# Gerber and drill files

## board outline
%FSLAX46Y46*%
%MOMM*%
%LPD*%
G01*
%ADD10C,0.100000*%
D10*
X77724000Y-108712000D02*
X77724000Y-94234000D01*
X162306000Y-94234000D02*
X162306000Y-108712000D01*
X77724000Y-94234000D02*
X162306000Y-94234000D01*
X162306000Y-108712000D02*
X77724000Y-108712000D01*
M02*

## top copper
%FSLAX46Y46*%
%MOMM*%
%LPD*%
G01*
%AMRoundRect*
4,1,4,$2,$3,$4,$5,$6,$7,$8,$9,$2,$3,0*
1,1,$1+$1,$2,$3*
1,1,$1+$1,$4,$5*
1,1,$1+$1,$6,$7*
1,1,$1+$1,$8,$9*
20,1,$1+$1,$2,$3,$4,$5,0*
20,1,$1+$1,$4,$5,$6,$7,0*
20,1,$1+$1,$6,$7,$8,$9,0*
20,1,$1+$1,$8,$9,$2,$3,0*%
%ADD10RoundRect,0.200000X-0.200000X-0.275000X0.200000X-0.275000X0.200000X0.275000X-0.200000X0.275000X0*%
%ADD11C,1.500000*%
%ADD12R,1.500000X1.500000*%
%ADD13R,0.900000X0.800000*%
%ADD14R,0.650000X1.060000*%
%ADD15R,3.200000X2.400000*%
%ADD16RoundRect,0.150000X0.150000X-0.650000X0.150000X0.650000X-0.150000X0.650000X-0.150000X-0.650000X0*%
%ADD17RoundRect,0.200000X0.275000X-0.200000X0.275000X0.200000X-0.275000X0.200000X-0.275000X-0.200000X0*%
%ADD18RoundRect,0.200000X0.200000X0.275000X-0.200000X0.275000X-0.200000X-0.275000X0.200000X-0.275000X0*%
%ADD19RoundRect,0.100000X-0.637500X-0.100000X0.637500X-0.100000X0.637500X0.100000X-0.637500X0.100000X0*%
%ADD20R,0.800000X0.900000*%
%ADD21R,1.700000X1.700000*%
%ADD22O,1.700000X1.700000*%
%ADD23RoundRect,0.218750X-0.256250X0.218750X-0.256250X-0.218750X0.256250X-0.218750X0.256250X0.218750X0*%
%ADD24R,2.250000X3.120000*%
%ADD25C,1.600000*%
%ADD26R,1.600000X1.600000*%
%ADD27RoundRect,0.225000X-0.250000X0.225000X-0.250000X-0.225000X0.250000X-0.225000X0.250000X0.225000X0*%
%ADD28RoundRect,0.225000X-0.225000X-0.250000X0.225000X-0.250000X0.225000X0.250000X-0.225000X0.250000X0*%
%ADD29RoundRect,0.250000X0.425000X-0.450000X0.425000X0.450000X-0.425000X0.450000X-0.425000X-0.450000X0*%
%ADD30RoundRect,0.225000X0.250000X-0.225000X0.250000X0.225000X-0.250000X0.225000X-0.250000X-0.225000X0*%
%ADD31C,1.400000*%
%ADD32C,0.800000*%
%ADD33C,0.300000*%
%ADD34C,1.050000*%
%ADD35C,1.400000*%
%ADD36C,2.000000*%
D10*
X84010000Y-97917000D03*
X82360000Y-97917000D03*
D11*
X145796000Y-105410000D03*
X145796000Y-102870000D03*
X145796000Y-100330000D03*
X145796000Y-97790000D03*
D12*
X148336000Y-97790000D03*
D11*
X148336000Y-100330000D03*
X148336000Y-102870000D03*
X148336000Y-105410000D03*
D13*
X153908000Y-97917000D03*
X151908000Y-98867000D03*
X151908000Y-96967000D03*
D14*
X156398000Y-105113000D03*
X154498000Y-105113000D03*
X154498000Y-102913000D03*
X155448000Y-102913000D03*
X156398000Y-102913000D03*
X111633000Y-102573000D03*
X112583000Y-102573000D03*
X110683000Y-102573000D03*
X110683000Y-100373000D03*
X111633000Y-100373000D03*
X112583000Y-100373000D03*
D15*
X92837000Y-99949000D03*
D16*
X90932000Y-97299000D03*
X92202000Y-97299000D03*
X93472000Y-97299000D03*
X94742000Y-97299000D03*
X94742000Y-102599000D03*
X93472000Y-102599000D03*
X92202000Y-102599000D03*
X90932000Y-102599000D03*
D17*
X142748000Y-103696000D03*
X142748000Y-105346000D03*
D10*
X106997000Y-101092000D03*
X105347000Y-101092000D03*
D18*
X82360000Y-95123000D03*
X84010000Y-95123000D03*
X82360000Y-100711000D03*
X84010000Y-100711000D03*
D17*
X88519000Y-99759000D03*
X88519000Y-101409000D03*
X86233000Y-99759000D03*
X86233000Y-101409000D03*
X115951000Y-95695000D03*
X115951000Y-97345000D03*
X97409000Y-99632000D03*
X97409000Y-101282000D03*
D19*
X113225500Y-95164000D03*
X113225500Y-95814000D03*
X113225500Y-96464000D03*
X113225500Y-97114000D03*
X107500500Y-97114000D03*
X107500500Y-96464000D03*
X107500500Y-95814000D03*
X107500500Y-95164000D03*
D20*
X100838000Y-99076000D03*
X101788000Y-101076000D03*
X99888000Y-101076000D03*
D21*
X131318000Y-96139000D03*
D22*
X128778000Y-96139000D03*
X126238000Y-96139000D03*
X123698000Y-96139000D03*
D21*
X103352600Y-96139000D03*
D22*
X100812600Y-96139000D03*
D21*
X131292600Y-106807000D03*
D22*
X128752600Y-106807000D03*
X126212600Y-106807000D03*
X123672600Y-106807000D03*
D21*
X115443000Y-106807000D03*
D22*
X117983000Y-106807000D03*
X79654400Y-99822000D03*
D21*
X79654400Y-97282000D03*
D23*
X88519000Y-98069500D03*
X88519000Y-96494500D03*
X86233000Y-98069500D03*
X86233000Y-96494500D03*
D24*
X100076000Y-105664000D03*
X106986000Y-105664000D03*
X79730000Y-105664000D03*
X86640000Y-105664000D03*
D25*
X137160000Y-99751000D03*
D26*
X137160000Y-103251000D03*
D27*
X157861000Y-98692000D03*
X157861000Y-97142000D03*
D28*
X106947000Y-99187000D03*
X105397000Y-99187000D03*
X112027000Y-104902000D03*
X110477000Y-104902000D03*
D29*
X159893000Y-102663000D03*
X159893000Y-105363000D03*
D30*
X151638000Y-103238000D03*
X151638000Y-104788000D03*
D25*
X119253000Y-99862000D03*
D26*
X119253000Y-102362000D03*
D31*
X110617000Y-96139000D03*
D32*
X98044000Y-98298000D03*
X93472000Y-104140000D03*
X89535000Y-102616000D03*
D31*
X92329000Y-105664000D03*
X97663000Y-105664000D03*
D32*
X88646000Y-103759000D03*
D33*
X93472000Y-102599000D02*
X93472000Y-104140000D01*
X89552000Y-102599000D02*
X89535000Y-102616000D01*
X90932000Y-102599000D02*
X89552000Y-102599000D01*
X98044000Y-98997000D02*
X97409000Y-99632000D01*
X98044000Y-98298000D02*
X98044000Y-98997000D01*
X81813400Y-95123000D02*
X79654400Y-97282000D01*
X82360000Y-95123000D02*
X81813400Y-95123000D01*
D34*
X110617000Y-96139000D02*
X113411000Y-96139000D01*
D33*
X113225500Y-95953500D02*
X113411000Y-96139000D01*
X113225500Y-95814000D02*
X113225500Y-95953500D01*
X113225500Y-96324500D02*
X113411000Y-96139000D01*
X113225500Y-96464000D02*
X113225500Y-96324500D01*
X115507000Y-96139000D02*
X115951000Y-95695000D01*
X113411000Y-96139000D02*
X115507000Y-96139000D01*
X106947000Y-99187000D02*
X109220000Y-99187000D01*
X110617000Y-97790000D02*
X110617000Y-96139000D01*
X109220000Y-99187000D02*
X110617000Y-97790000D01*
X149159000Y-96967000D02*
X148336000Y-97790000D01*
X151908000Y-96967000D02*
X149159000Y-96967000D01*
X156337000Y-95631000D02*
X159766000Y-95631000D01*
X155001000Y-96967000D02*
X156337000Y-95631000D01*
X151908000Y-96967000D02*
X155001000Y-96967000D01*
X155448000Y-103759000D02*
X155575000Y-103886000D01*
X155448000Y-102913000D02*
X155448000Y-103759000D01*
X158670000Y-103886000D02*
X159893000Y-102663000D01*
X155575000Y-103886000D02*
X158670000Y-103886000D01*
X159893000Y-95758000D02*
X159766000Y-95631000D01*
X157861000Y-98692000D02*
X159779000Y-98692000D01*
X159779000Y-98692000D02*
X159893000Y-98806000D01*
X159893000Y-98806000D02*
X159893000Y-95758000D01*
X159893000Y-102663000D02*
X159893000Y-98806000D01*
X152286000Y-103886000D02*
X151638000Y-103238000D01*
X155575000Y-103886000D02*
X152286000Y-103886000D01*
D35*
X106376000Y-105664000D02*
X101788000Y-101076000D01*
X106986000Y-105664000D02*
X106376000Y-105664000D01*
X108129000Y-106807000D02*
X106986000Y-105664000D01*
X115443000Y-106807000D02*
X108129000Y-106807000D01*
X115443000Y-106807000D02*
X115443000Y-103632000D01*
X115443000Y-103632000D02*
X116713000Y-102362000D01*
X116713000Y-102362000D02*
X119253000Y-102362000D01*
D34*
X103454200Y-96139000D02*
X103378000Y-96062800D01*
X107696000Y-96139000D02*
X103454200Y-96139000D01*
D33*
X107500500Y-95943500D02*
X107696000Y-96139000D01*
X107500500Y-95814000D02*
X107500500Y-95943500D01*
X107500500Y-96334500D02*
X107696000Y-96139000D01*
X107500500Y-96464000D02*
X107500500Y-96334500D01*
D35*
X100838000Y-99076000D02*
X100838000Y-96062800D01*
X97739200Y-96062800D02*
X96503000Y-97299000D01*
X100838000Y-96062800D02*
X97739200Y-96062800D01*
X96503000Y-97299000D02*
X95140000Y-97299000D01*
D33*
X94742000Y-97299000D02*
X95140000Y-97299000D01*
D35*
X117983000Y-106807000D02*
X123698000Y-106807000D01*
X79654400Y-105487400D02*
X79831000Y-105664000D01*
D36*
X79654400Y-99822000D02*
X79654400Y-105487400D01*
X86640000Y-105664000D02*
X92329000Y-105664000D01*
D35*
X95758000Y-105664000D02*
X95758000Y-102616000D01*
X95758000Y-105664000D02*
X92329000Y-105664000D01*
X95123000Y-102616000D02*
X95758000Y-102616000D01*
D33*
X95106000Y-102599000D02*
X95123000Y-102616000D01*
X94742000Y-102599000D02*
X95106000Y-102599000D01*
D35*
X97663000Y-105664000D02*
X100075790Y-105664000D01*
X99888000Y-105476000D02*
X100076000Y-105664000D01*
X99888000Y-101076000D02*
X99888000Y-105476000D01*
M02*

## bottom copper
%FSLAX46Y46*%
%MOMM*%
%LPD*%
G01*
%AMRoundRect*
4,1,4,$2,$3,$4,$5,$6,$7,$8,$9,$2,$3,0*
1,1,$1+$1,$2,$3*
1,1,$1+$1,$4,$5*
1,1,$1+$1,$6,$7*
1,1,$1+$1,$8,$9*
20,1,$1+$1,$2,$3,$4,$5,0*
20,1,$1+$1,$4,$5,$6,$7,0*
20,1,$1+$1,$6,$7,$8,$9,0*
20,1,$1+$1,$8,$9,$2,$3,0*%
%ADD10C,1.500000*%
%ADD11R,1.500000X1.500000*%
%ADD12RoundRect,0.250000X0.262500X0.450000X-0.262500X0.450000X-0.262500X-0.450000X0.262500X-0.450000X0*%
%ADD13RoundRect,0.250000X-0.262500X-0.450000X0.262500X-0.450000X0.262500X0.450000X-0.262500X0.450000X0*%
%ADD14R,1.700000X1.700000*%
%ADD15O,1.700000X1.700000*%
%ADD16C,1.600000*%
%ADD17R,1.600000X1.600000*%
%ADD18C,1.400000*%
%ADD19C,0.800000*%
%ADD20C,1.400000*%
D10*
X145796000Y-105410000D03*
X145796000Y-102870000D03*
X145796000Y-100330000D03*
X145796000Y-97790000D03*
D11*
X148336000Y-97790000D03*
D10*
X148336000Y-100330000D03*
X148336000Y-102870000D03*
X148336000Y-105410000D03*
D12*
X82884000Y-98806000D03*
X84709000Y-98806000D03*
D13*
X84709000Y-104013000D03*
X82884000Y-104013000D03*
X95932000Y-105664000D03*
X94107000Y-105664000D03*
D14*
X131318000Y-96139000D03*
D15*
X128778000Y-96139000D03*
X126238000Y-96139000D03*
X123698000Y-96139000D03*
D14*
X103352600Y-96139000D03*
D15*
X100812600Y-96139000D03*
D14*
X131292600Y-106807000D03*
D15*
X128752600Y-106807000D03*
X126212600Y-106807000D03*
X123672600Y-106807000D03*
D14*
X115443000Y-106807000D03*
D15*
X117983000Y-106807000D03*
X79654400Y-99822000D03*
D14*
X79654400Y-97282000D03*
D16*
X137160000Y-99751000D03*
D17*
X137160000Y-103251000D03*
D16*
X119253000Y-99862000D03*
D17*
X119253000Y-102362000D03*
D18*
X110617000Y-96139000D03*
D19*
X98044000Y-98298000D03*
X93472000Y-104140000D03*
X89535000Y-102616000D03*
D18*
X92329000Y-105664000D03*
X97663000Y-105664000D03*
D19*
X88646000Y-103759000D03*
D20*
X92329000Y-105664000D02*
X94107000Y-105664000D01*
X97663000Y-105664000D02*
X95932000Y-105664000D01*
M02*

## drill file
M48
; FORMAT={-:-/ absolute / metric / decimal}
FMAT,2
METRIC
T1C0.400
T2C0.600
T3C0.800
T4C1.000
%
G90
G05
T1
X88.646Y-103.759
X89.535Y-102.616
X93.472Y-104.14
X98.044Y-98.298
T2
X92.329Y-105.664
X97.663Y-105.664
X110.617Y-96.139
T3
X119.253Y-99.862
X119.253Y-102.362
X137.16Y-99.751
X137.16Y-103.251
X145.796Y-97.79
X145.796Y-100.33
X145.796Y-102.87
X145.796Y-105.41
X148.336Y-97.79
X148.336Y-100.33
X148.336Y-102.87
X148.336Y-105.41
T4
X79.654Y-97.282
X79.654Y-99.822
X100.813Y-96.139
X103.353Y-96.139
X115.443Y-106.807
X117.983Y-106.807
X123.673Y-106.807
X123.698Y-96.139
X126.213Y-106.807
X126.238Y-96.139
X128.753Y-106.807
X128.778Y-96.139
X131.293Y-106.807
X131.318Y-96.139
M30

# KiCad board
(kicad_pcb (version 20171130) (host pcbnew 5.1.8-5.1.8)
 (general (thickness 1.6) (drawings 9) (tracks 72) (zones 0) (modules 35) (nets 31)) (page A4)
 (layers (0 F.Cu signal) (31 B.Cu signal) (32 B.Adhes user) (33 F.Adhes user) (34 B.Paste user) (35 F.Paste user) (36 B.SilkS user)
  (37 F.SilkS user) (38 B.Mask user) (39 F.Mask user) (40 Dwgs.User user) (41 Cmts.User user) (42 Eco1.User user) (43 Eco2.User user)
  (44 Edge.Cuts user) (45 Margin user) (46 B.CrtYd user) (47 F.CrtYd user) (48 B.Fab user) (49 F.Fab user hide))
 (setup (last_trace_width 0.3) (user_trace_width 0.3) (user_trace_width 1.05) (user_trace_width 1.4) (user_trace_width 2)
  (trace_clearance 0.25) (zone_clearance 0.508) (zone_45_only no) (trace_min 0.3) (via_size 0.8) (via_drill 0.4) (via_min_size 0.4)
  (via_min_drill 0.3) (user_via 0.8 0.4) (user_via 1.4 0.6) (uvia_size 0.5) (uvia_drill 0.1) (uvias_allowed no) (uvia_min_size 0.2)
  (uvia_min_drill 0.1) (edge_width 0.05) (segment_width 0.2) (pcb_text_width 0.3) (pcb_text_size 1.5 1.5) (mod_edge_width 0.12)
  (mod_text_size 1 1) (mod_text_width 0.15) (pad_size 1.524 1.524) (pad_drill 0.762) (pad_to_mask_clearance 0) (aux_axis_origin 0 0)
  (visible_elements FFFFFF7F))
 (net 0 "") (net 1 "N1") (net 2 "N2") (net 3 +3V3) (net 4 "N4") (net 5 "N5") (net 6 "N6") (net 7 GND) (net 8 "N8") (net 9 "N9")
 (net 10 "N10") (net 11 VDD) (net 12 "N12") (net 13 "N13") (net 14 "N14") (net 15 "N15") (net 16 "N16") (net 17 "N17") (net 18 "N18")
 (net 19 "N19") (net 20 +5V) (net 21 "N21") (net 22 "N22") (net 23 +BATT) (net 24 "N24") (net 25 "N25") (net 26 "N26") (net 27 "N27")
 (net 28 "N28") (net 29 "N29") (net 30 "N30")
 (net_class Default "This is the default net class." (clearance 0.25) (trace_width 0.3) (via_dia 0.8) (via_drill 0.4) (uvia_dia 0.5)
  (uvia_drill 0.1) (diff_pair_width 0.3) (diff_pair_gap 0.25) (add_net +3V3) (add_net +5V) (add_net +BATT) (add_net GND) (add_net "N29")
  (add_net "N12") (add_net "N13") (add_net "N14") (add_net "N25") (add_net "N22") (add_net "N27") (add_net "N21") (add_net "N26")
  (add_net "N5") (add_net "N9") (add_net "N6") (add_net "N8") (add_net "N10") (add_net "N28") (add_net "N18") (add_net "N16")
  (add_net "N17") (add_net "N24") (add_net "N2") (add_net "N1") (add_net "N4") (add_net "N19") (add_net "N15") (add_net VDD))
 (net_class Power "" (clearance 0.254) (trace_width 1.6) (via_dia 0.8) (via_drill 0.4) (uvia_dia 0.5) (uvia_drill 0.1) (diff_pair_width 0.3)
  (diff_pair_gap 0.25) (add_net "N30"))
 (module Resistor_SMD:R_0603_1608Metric (layer F.Cu) (at 83.185 97.917)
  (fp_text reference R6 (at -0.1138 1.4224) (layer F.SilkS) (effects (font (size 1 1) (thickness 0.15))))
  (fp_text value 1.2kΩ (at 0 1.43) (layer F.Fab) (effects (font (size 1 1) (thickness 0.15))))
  (pad 2 smd roundrect (at 0.825 0) (size 0.8 0.95) (layers F.Cu F.Paste F.Mask) (roundrect_rratio 0.25) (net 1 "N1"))
  (pad 1 smd roundrect (at -0.825 0) (size 0.8 0.95) (layers F.Cu F.Paste F.Mask) (roundrect_rratio 0.25) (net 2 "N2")))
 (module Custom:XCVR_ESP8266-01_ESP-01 (layer F.Cu) (at 156.646 101.6 270)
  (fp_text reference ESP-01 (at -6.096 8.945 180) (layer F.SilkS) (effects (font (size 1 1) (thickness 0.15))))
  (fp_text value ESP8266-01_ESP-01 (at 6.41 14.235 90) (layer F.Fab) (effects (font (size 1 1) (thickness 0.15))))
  (pad 8 thru_hole circle (at 3.81 10.85 270) (size 1.5 1.5) (drill 0.8) (layers *.Cu *.Mask) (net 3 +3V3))
  (pad 7 thru_hole circle (at 1.27 10.85 270) (size 1.5 1.5) (drill 0.8) (layers *.Cu *.Mask) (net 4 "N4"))
  (pad 6 thru_hole circle (at -1.27 10.85 270) (size 1.5 1.5) (drill 0.8) (layers *.Cu *.Mask) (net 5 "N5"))
  (pad 5 thru_hole circle (at -3.81 10.85 270) (size 1.5 1.5) (drill 0.8) (layers *.Cu *.Mask) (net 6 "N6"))
  (pad 1 thru_hole rect (at -3.81 8.31 270) (size 1.5 1.5) (drill 0.8) (layers *.Cu *.Mask) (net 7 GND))
  (pad 2 thru_hole circle (at -1.27 8.31 270) (size 1.5 1.5) (drill 0.8) (layers *.Cu *.Mask) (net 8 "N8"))
  (pad 3 thru_hole circle (at 1.27 8.31 270) (size 1.5 1.5) (drill 0.8) (layers *.Cu *.Mask) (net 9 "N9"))
  (pad 4 thru_hole circle (at 3.81 8.31 270) (size 1.5 1.5) (drill 0.8) (layers *.Cu *.Mask) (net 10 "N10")))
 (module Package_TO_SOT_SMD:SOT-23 (layer F.Cu) (at 152.908 97.917)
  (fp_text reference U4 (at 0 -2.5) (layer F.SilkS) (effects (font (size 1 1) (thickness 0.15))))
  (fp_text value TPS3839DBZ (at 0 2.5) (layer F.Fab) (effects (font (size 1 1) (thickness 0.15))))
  (pad 3 smd rect (at 1 0) (size 0.9 0.8) (layers F.Cu F.Paste F.Mask) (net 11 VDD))
  (pad 2 smd rect (at -1 0.95) (size 0.9 0.8) (layers F.Cu F.Paste F.Mask) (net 5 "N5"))
  (pad 1 smd rect (at -1 -0.95) (size 0.9 0.8) (layers F.Cu F.Paste F.Mask) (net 7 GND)))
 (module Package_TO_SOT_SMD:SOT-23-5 (layer F.Cu) (at 155.448 104.013 270)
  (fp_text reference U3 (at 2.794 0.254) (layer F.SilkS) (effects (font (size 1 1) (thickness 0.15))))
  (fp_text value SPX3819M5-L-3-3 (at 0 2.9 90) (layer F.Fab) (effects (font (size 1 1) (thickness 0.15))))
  (pad 5 smd rect (at 1.1 -0.95 270) (size 1.06 0.65) (layers F.Cu F.Paste F.Mask) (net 3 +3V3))
  (pad 4 smd rect (at 1.1 0.95 270) (size 1.06 0.65) (layers F.Cu F.Paste F.Mask) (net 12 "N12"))
  (pad 3 smd rect (at -1.1 0.95 270) (size 1.06 0.65) (layers F.Cu F.Paste F.Mask) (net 11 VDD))
  (pad 2 smd rect (at -1.1 0 270) (size 1.06 0.65) (layers F.Cu F.Paste F.Mask) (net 7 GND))
  (pad 1 smd rect (at -1.1 -0.95 270) (size 1.06 0.65) (layers F.Cu F.Paste F.Mask) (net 11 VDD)))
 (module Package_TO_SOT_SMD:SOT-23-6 (layer F.Cu) (at 111.633 101.473 270)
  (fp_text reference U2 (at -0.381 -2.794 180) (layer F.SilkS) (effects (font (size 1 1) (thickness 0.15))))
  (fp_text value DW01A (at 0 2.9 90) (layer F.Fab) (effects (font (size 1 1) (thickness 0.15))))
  (pad 5 smd rect (at 1.1 0 270) (size 1.06 0.65) (layers F.Cu F.Paste F.Mask) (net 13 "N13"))
  (pad 6 smd rect (at 1.1 -0.95 270) (size 1.06 0.65) (layers F.Cu F.Paste F.Mask) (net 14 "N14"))
  (pad 4 smd rect (at 1.1 0.95 270) (size 1.06 0.65) (layers F.Cu F.Paste F.Mask) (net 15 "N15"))
  (pad 3 smd rect (at -1.1 0.95 270) (size 1.06 0.65) (layers F.Cu F.Paste F.Mask) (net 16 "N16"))
  (pad 2 smd rect (at -1.1 0 270) (size 1.06 0.65) (layers F.Cu F.Paste F.Mask) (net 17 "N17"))
  (pad 1 smd rect (at -1.1 -0.95 270) (size 1.06 0.65) (layers F.Cu F.Paste F.Mask) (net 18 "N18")))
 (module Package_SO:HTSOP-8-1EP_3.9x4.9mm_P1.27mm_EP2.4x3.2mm (layer F.Cu) (at 92.837 99.949 90)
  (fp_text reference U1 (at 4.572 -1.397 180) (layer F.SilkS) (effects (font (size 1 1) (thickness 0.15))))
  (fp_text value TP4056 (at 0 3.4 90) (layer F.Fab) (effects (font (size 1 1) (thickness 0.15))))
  (pad "" smd roundrect (at 0.6 0.8 90) (size 0.97 1.29) (layers F.Paste) (roundrect_rratio 0.25))
  (pad "" smd roundrect (at 0.6 -0.8 90) (size 0.97 1.29) (layers F.Paste) (roundrect_rratio 0.25))
  (pad "" smd roundrect (at -0.6 0.8 90) (size 0.97 1.29) (layers F.Paste) (roundrect_rratio 0.25))
  (pad "" smd roundrect (at -0.6 -0.8 90) (size 0.97 1.29) (layers F.Paste) (roundrect_rratio 0.25))
  (pad 9 smd rect (at 0 0 90) (size 2.4 3.2) (layers F.Cu F.Mask) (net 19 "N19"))
  (pad 8 smd roundrect (at 2.65 -1.905 90) (size 1.6 0.6) (layers F.Cu F.Paste F.Mask) (roundrect_rratio 0.25) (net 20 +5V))
  (pad 7 smd roundrect (at 2.65 -0.635 90) (size 1.6 0.6) (layers F.Cu F.Paste F.Mask) (roundrect_rratio 0.25) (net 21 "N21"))
  (pad 6 smd roundrect (at 2.65 0.635 90) (size 1.6 0.6) (layers F.Cu F.Paste F.Mask) (roundrect_rratio 0.25) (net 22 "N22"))
  (pad 5 smd roundrect (at 2.65 1.905 90) (size 1.6 0.6) (layers F.Cu F.Paste F.Mask) (roundrect_rratio 0.25) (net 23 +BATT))
  (pad 4 smd roundrect (at -2.65 1.905 90) (size 1.6 0.6) (layers F.Cu F.Paste F.Mask) (roundrect_rratio 0.25) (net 20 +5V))
  (pad 3 smd roundrect (at -2.65 0.635 90) (size 1.6 0.6) (layers F.Cu F.Paste F.Mask) (roundrect_rratio 0.25) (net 7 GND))
  (pad 2 smd roundrect (at -2.65 -0.635 90) (size 1.6 0.6) (layers F.Cu F.Paste F.Mask) (roundrect_rratio 0.25) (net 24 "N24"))
  (pad 1 smd roundrect (at -2.65 -1.905 90) (size 1.6 0.6) (layers F.Cu F.Paste F.Mask) (roundrect_rratio 0.25) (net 7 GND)))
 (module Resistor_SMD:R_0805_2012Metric (layer B.Cu) (at 83.7965 98.806 180)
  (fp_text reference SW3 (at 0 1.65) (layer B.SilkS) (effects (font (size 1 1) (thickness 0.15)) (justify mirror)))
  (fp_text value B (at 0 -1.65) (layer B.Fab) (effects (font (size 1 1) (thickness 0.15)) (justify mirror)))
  (pad 2 smd roundrect (at 0.9125 0 180) (size 1.025 1.4) (layers B.Cu B.Paste B.Mask) (roundrect_rratio 0.243902) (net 2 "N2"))
  (pad 1 smd roundrect (at -0.9125 0 180) (size 1.025 1.4) (layers B.Cu B.Paste B.Mask) (roundrect_rratio 0.243902) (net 1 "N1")))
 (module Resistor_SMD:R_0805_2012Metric (layer B.Cu) (at 83.7965 104.013)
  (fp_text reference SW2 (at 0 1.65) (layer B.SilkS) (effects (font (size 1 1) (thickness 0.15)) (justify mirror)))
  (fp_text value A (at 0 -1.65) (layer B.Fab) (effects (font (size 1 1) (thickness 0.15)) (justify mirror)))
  (pad 2 smd roundrect (at 0.9125 0) (size 1.025 1.4) (layers B.Cu B.Paste B.Mask) (roundrect_rratio 0.243902) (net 24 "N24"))
  (pad 1 smd roundrect (at -0.9125 0) (size 1.025 1.4) (layers B.Cu B.Paste B.Mask) (roundrect_rratio 0.243902) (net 2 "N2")))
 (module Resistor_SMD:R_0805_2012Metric (layer B.Cu) (at 95.0195 105.664)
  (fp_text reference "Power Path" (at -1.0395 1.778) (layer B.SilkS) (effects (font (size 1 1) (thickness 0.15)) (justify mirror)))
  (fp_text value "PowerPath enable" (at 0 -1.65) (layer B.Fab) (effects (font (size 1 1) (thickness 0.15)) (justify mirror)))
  (pad 2 smd roundrect (at 0.9125 0) (size 1.025 1.4) (layers B.Cu B.Paste B.Mask) (roundrect_rratio 0.243902) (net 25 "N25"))
  (pad 1 smd roundrect (at -0.9125 0) (size 1.025 1.4) (layers B.Cu B.Paste B.Mask) (roundrect_rratio 0.243902) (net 20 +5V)))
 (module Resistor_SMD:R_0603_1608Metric (layer F.Cu) (at 142.748 104.521 90)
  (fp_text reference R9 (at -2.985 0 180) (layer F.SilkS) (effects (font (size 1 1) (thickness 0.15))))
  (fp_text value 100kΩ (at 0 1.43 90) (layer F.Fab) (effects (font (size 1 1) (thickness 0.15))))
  (pad 2 smd roundrect (at 0.825 0 90) (size 0.8 0.95) (layers F.Cu F.Paste F.Mask) (roundrect_rratio 0.25) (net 4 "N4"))
  (pad 1 smd roundrect (at -0.825 0 90) (size 0.8 0.95) (layers F.Cu F.Paste F.Mask) (roundrect_rratio 0.25) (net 3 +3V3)))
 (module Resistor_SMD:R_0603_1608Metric (layer F.Cu) (at 106.172 101.092)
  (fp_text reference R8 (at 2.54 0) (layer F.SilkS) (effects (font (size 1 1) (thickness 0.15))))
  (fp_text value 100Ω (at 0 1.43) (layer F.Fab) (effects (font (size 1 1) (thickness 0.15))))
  (pad 2 smd roundrect (at 0.825 0) (size 0.8 0.95) (layers F.Cu F.Paste F.Mask) (roundrect_rratio 0.25) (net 13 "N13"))
  (pad 1 smd roundrect (at -0.825 0) (size 0.8 0.95) (layers F.Cu F.Paste F.Mask) (roundrect_rratio 0.25) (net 23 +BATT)))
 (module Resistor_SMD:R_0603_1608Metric (layer F.Cu) (at 83.185 95.123 180)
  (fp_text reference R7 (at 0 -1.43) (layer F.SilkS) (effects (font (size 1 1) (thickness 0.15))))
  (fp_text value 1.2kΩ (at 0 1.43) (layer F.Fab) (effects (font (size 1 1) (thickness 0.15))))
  (pad 2 smd roundrect (at 0.825 0 180) (size 0.8 0.95) (layers F.Cu F.Paste F.Mask) (roundrect_rratio 0.25) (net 7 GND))
  (pad 1 smd roundrect (at -0.825 0 180) (size 0.8 0.95) (layers F.Cu F.Paste F.Mask) (roundrect_rratio 0.25) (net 1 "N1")))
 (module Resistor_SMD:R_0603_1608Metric (layer F.Cu) (at 83.185 100.711 180)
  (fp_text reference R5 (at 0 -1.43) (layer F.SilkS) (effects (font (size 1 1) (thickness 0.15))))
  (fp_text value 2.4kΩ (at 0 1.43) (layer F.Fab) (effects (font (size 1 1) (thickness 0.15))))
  (pad 2 smd roundrect (at 0.825 0 180) (size 0.8 0.95) (layers F.Cu F.Paste F.Mask) (roundrect_rratio 0.25) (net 2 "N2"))
  (pad 1 smd roundrect (at -0.825 0 180) (size 0.8 0.95) (layers F.Cu F.Paste F.Mask) (roundrect_rratio 0.25) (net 24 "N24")))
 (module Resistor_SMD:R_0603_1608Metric (layer F.Cu) (at 88.519 100.584 90)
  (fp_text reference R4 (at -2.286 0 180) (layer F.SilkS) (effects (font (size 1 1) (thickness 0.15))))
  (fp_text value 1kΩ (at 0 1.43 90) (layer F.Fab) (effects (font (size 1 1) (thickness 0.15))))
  (pad 2 smd roundrect (at 0.825 0 90) (size 0.8 0.95) (layers F.Cu F.Paste F.Mask) (roundrect_rratio 0.25) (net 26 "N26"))
  (pad 1 smd roundrect (at -0.825 0 90) (size 0.8 0.95) (layers F.Cu F.Paste F.Mask) (roundrect_rratio 0.25) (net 20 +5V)))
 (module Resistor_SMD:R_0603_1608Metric (layer F.Cu) (at 86.233 100.584 90)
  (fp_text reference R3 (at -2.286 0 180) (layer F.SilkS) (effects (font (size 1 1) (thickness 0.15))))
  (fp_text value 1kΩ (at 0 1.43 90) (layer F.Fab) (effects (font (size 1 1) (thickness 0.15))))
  (pad 2 smd roundrect (at 0.825 0 90) (size 0.8 0.95) (layers F.Cu F.Paste F.Mask) (roundrect_rratio 0.25) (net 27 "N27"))
  (pad 1 smd roundrect (at -0.825 0 90) (size 0.8 0.95) (layers F.Cu F.Paste F.Mask) (roundrect_rratio 0.25) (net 20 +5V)))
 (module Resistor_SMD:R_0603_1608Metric (layer F.Cu) (at 115.951 96.52 90)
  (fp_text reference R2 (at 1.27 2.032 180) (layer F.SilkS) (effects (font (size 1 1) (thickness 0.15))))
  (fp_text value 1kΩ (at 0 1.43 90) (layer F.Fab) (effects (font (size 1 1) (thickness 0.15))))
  (pad 2 smd roundrect (at 0.825 0 90) (size 0.8 0.95) (layers F.Cu F.Paste F.Mask) (roundrect_rratio 0.25) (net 7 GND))
  (pad 1 smd roundrect (at -0.825 0 90) (size 0.8 0.95) (layers F.Cu F.Paste F.Mask) (roundrect_rratio 0.25) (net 17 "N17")))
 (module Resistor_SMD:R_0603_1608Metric (layer F.Cu) (at 97.409 100.457 90)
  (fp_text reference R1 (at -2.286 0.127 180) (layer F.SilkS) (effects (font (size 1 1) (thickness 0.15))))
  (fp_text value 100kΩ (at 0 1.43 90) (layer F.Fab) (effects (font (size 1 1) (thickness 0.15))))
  (pad 2 smd roundrect (at 0.825 0 90) (size 0.8 0.95) (layers F.Cu F.Paste F.Mask) (roundrect_rratio 0.25) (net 7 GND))
  (pad 1 smd roundrect (at -0.825 0 90) (size 0.8 0.95) (layers F.Cu F.Paste F.Mask) (roundrect_rratio 0.25) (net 25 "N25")))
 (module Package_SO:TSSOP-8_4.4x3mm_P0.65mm (layer F.Cu) (at 110.363 96.139)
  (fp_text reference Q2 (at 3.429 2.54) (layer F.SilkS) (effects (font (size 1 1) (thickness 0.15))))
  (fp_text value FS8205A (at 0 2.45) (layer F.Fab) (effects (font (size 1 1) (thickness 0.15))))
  (pad 8 smd roundrect (at 2.8625 -0.975) (size 1.475 0.4) (layers F.Cu F.Paste F.Mask) (roundrect_rratio 0.25) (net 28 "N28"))
  (pad 7 smd roundrect (at 2.8625 -0.325) (size 1.475 0.4) (layers F.Cu F.Paste F.Mask) (roundrect_rratio 0.25) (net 7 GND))
  (pad 6 smd roundrect (at 2.8625 0.325) (size 1.475 0.4) (layers F.Cu F.Paste F.Mask) (roundrect_rratio 0.25) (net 7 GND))
  (pad 5 smd roundrect (at 2.8625 0.975) (size 1.475 0.4) (layers F.Cu F.Paste F.Mask) (roundrect_rratio 0.25) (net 16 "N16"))
  (pad 4 smd roundrect (at -2.8625 0.975) (size 1.475 0.4) (layers F.Cu F.Paste F.Mask) (roundrect_rratio 0.25) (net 18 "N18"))
  (pad 3 smd roundrect (at -2.8625 0.325) (size 1.475 0.4) (layers F.Cu F.Paste F.Mask) (roundrect_rratio 0.25) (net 14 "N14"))
  (pad 2 smd roundrect (at -2.8625 -0.325) (size 1.475 0.4) (layers F.Cu F.Paste F.Mask) (roundrect_rratio 0.25) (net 14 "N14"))
  (pad 1 smd roundrect (at -2.8625 -0.975) (size 1.475 0.4) (layers F.Cu F.Paste F.Mask) (roundrect_rratio 0.25) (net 28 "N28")))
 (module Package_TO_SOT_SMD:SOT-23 (layer F.Cu) (at 100.838 100.076 90)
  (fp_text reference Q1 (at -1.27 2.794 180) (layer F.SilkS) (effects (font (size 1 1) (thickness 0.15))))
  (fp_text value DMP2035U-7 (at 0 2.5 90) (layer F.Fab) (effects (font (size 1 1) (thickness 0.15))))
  (pad 3 smd rect (at 1 0 90) (size 0.9 0.8) (layers F.Cu F.Paste F.Mask) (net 23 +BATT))
  (pad 2 smd rect (at -1 0.95 90) (size 0.9 0.8) (layers F.Cu F.Paste F.Mask) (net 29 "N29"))
  (pad 1 smd rect (at -1 -0.95 90) (size 0.9 0.8) (layers F.Cu F.Paste F.Mask) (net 25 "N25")))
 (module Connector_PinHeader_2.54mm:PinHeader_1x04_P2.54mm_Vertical (layer F.Cu) (at 131.318 96.139 270)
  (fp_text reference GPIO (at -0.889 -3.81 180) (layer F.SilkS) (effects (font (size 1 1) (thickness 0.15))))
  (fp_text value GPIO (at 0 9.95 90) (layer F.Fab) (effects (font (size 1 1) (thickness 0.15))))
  (pad 1 thru_hole rect (at 0 0 270) (size 1.7 1.7) (drill 1) (layers *.Cu *.Mask) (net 9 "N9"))
  (pad 2 thru_hole oval (at 0 2.54 270) (size 1.7 1.7) (drill 1) (layers *.Cu *.Mask) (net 6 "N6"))
  (pad 3 thru_hole oval (at 0 5.08 270) (size 1.7 1.7) (drill 1) (layers *.Cu *.Mask) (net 8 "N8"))
  (pad 4 thru_hole oval (at 0 7.62 270) (size 1.7 1.7) (drill 1) (layers *.Cu *.Mask) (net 10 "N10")))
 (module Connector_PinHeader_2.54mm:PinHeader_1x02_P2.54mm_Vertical (layer F.Cu) (at 103.3526 96.139 270)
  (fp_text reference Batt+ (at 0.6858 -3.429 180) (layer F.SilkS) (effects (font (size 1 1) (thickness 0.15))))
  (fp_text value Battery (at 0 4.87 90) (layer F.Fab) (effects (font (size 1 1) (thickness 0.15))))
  (pad 1 thru_hole rect (at 0 0 270) (size 1.7 1.7) (drill 1) (layers *.Cu *.Mask) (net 14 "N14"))
  (pad 2 thru_hole oval (at 0 2.54 270) (size 1.7 1.7) (drill 1) (layers *.Cu *.Mask) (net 23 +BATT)))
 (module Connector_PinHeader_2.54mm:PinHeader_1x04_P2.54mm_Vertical (layer F.Cu) (at 131.2926 106.807 270)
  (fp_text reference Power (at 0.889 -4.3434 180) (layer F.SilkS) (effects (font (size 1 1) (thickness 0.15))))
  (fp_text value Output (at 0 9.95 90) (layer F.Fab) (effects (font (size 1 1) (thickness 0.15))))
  (pad 1 thru_hole rect (at 0 0 270) (size 1.7 1.7) (drill 1) (layers *.Cu *.Mask) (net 7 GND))
  (pad 2 thru_hole oval (at 0 2.54 270) (size 1.7 1.7) (drill 1) (layers *.Cu *.Mask) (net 5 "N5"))
  (pad 3 thru_hole oval (at 0 5.08 270) (size 1.7 1.7) (drill 1) (layers *.Cu *.Mask) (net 3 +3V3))
  (pad 4 thru_hole oval (at 0 7.62 270) (size 1.7 1.7) (drill 1) (layers *.Cu *.Mask) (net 11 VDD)))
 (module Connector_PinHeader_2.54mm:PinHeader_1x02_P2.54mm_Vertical (layer F.Cu) (at 115.443 106.807 90)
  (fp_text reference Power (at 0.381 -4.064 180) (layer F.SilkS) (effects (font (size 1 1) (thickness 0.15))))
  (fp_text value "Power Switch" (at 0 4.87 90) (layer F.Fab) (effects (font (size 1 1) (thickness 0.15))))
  (pad 1 thru_hole rect (at 0 0 90) (size 1.7 1.7) (drill 1) (layers *.Cu *.Mask) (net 29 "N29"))
  (pad 2 thru_hole oval (at 0 2.54 90) (size 1.7 1.7) (drill 1) (layers *.Cu *.Mask) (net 11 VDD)))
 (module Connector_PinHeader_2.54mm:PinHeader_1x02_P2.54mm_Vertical (layer F.Cu) (at 79.6544 97.282)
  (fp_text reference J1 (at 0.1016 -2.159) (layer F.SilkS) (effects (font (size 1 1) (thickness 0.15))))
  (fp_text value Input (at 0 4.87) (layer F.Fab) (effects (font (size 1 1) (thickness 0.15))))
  (pad 2 thru_hole oval (at 0 2.54) (size 1.7 1.7) (drill 1) (layers *.Cu *.Mask) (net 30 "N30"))
  (pad 1 thru_hole rect (at 0 0) (size 1.7 1.7) (drill 1) (layers *.Cu *.Mask) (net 7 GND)))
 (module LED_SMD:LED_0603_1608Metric (layer F.Cu) (at 88.519 97.282 270)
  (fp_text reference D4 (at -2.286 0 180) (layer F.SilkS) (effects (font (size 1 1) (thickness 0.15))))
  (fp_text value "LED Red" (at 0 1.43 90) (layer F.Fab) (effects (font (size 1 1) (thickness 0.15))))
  (pad 2 smd roundrect (at 0.7875 0 270) (size 0.875 0.95) (layers F.Cu F.Paste F.Mask) (roundrect_rratio 0.25) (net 26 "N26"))
  (pad 1 smd roundrect (at -0.7875 0 270) (size 0.875 0.95) (layers F.Cu F.Paste F.Mask) (roundrect_rratio 0.25) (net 21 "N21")))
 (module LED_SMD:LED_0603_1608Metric (layer F.Cu) (at 86.233 97.282 270)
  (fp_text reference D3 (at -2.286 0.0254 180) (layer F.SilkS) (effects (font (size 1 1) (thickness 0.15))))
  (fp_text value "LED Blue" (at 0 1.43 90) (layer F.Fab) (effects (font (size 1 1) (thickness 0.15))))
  (pad 2 smd roundrect (at 0.7875 0 270) (size 0.875 0.95) (layers F.Cu F.Paste F.Mask) (roundrect_rratio 0.25) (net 27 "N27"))
  (pad 1 smd roundrect (at -0.7875 0 270) (size 0.875 0.95) (layers F.Cu F.Paste F.Mask) (roundrect_rratio 0.25) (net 22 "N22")))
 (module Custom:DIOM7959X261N (layer F.Cu) (at 103.531 105.664 180)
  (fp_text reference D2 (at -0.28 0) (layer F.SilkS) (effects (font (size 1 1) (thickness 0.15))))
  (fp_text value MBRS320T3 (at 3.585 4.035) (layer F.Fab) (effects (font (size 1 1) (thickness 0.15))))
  (pad A smd rect (at 3.455 0 180) (size 2.25 3.12) (layers F.Cu F.Paste F.Mask) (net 25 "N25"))
  (pad C smd rect (at -3.455 0 180) (size 2.25 3.12) (layers F.Cu F.Paste F.Mask) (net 29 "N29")))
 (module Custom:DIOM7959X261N (layer F.Cu) (at 83.185 105.664 180)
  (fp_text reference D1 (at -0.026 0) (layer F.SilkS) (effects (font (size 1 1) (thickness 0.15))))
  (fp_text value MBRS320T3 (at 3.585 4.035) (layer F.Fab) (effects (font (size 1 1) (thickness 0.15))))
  (pad A smd rect (at 3.455 0 180) (size 2.25 3.12) (layers F.Cu F.Paste F.Mask) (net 30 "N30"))
  (pad C smd rect (at -3.455 0 180) (size 2.25 3.12) (layers F.Cu F.Paste F.Mask) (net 20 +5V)))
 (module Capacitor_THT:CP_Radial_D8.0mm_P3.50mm (layer F.Cu) (at 137.16 103.251 90)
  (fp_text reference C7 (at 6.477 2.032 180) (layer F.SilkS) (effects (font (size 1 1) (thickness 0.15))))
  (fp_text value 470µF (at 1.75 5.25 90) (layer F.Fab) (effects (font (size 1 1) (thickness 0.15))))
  (pad 2 thru_hole circle (at 3.5 0 90) (size 1.6 1.6) (drill 0.8) (layers *.Cu *.Mask) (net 7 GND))
  (pad 1 thru_hole rect (at 0 0 90) (size 1.6 1.6) (drill 0.8) (layers *.Cu *.Mask) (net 3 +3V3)))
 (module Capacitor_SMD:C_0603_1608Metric (layer F.Cu) (at 157.861 97.917 270)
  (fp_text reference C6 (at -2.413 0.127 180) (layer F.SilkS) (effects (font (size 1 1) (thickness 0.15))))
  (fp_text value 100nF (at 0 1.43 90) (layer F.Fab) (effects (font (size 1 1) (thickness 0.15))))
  (pad 2 smd roundrect (at 0.775 0 270) (size 0.9 0.95) (layers F.Cu F.Paste F.Mask) (roundrect_rratio 0.25) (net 7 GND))
  (pad 1 smd roundrect (at -0.775 0 270) (size 0.9 0.95) (layers F.Cu F.Paste F.Mask) (roundrect_rratio 0.25) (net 11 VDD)))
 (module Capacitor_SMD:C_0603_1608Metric (layer F.Cu) (at 106.172 99.187)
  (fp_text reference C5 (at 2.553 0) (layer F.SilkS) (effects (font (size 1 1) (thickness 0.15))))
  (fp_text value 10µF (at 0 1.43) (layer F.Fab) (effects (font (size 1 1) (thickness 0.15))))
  (pad 2 smd roundrect (at 0.775 0) (size 0.9 0.95) (layers F.Cu F.Paste F.Mask) (roundrect_rratio 0.25) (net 7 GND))
  (pad 1 smd roundrect (at -0.775 0) (size 0.9 0.95) (layers F.Cu F.Paste F.Mask) (roundrect_rratio 0.25) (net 23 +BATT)))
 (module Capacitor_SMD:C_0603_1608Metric (layer F.Cu) (at 111.252 104.902)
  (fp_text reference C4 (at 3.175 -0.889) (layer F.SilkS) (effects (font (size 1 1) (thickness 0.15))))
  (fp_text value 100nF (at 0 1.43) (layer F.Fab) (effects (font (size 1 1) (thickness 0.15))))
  (pad 2 smd roundrect (at 0.775 0) (size 0.9 0.95) (layers F.Cu F.Paste F.Mask) (roundrect_rratio 0.25) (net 14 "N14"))
  (pad 1 smd roundrect (at -0.775 0) (size 0.9 0.95) (layers F.Cu F.Paste F.Mask) (roundrect_rratio 0.25) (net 13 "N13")))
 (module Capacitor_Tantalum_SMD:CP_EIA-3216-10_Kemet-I (layer F.Cu) (at 159.893 104.013 90)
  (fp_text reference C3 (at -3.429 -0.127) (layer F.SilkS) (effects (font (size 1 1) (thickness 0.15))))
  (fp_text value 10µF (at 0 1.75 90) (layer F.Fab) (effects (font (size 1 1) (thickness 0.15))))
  (pad 2 smd roundrect (at 1.35 0 90) (size 1.4 1.35) (layers F.Cu F.Paste F.Mask) (roundrect_rratio 0.185185) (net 7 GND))
  (pad 1 smd roundrect (at -1.35 0 90) (size 1.4 1.35) (layers F.Cu F.Paste F.Mask) (roundrect_rratio 0.185185) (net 3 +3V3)))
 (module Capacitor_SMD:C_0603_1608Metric (layer F.Cu) (at 151.638 104.013 90)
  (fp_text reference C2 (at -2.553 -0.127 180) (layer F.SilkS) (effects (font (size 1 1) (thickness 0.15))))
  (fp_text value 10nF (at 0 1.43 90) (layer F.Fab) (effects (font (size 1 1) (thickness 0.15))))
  (pad 2 smd roundrect (at 0.775 0 90) (size 0.9 0.95) (layers F.Cu F.Paste F.Mask) (roundrect_rratio 0.25) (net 7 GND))
  (pad 1 smd roundrect (at -0.775 0 90) (size 0.9 0.95) (layers F.Cu F.Paste F.Mask) (roundrect_rratio 0.25) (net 12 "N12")))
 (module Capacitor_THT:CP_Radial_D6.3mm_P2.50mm (layer F.Cu) (at 119.253 102.362 90)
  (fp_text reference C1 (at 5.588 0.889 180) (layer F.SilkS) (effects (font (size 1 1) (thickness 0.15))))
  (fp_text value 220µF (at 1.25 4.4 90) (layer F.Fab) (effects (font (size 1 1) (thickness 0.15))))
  (pad 2 thru_hole circle (at 2.5 0 90) (size 1.6 1.6) (drill 0.8) (layers *.Cu *.Mask) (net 7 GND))
  (pad 1 thru_hole rect (at 0 0 90) (size 1.6 1.6) (drill 0.8) (layers *.Cu *.Mask) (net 29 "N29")))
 (gr_line (start 77.724 108.712) (end 77.724 94.234) (layer Edge.Cuts) (width 0.1))
 (gr_line (start 162.306 94.234) (end 162.306 108.712) (layer Edge.Cuts) (width 0.1))
 (gr_line (start 77.724 94.234) (end 162.306 94.234) (layer Edge.Cuts) (width 0.1))
 (gr_line (start 162.306 108.712) (end 77.724 108.712) (layer Edge.Cuts) (width 0.1))
 (via (at 110.617 96.139) (size 1.4) (drill 0.6) (layers F.Cu B.Cu) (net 7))
 (via (at 98.044 98.298) (size 0.8) (drill 0.4) (layers F.Cu B.Cu) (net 7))
 (via (at 93.472 104.14) (size 0.8) (drill 0.4) (layers F.Cu B.Cu) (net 7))
 (via (at 89.535 102.616) (size 0.8) (drill 0.4) (layers F.Cu B.Cu) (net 7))
 (segment (start 93.472 102.599) (end 93.472 104.14) (width 0.3) (layer F.Cu) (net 7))
 (segment (start 89.552 102.599) (end 89.535 102.616) (width 0.3) (layer F.Cu) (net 7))
 (segment (start 90.932 102.599) (end 89.552 102.599) (width 0.3) (layer F.Cu) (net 7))
 (segment (start 98.044 98.997) (end 97.409 99.632) (width 0.3) (layer F.Cu) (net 7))
 (segment (start 98.044 98.298) (end 98.044 98.997) (width 0.3) (layer F.Cu) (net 7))
 (segment (start 81.8134 95.123) (end 79.6544 97.282) (width 0.3) (layer F.Cu) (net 7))
 (segment (start 82.36 95.123) (end 81.8134 95.123) (width 0.3) (layer F.Cu) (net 7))
 (segment (start 110.617 96.139) (end 113.411 96.139) (width 1.05) (layer F.Cu) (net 7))
 (segment (start 113.2255 95.9535) (end 113.411 96.139) (width 0.3) (layer F.Cu) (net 7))
 (segment (start 113.2255 95.814) (end 113.2255 95.9535) (width 0.3) (layer F.Cu) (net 7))
 (segment (start 113.2255 96.3245) (end 113.411 96.139) (width 0.3) (layer F.Cu) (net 7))
 (segment (start 113.2255 96.464) (end 113.2255 96.3245) (width 0.3) (layer F.Cu) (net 7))
 (segment (start 115.507 96.139) (end 115.951 95.695) (width 0.3) (layer F.Cu) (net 7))
 (segment (start 113.411 96.139) (end 115.507 96.139) (width 0.3) (layer F.Cu) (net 7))
 (segment (start 106.947 99.187) (end 109.22 99.187) (width 0.3) (layer F.Cu) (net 7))
 (segment (start 110.617 97.79) (end 110.617 96.139) (width 0.3) (layer F.Cu) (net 7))
 (segment (start 109.22 99.187) (end 110.617 97.79) (width 0.3) (layer F.Cu) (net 7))
 (segment (start 149.159 96.967) (end 148.336 97.79) (width 0.3) (layer F.Cu) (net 7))
 (segment (start 151.908 96.967) (end 149.159 96.967) (width 0.3) (layer F.Cu) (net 7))
 (segment (start 156.337 95.631) (end 159.766 95.631) (width 0.3) (layer F.Cu) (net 7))
 (segment (start 155.001 96.967) (end 156.337 95.631) (width 0.3) (layer F.Cu) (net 7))
 (segment (start 151.908 96.967) (end 155.001 96.967) (width 0.3) (layer F.Cu) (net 7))
 (segment (start 155.448 103.759) (end 155.575 103.886) (width 0.3) (layer F.Cu) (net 7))
 (segment (start 155.448 102.913) (end 155.448 103.759) (width 0.3) (layer F.Cu) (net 7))
 (segment (start 158.67 103.886) (end 159.893 102.663) (width 0.3) (layer F.Cu) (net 7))
 (segment (start 155.575 103.886) (end 158.67 103.886) (width 0.3) (layer F.Cu) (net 7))
 (segment (start 159.893 95.758) (end 159.766 95.631) (width 0.3) (layer F.Cu) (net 7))
 (segment (start 157.861 98.692) (end 159.779 98.692) (width 0.3) (layer F.Cu) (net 7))
 (segment (start 159.779 98.692) (end 159.893 98.806) (width 0.3) (layer F.Cu) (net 7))
 (segment (start 159.893 98.806) (end 159.893 95.758) (width 0.3) (layer F.Cu) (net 7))
 (segment (start 159.893 102.663) (end 159.893 98.806) (width 0.3) (layer F.Cu) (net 7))
 (segment (start 152.286 103.886) (end 151.638 103.238) (width 0.3) (layer F.Cu) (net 7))
 (segment (start 155.575 103.886) (end 152.286 103.886) (width 0.3) (layer F.Cu) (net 7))
 (segment (start 106.376 105.664) (end 101.788 101.076) (width 1.4) (layer F.Cu) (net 29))
 (segment (start 106.986 105.664) (end 106.376 105.664) (width 1.4) (layer F.Cu) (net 29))
 (segment (start 108.129 106.807) (end 106.986 105.664) (width 1.4) (layer F.Cu) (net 29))
 (segment (start 115.443 106.807) (end 108.129 106.807) (width 1.4) (layer F.Cu) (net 29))
 (segment (start 115.443 106.807) (end 115.443 103.632) (width 1.4) (layer F.Cu) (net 29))
 (segment (start 115.443 103.632) (end 116.713 102.362) (width 1.4) (layer F.Cu) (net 29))
 (segment (start 116.713 102.362) (end 119.253 102.362) (width 1.4) (layer F.Cu) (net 29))
 (segment (start 103.4542 96.139) (end 103.378 96.0628) (width 1.05) (layer F.Cu) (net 14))
 (segment (start 107.696 96.139) (end 103.4542 96.139) (width 1.05) (layer F.Cu) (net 14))
 (segment (start 107.5005 95.9435) (end 107.696 96.139) (width 0.3) (layer F.Cu) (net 14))
 (segment (start 107.5005 95.814) (end 107.5005 95.9435) (width 0.3) (layer F.Cu) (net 14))
 (segment (start 107.5005 96.3345) (end 107.696 96.139) (width 0.3) (layer F.Cu) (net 14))
 (segment (start 107.5005 96.464) (end 107.5005 96.3345) (width 0.3) (layer F.Cu) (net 14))
 (segment (start 100.838 99.076) (end 100.838 96.0628) (width 1.4) (layer F.Cu) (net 23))
 (segment (start 97.7392 96.0628) (end 96.503 97.299) (width 1.4) (layer F.Cu) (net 23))
 (segment (start 100.838 96.0628) (end 97.7392 96.0628) (width 1.4) (layer F.Cu) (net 23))
 (segment (start 96.503 97.299) (end 95.14 97.299) (width 1.4) (layer F.Cu) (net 23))
 (segment (start 94.742 97.299) (end 95.14 97.299) (width 0.3) (layer F.Cu) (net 23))
 (segment (start 117.983 106.807) (end 123.698 106.807) (width 1.4) (layer F.Cu) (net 11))
 (segment (start 79.6544 105.4874) (end 79.831 105.664) (width 1.4) (layer F.Cu) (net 30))
 (segment (start 79.6544 99.822) (end 79.6544 105.4874) (width 2) (layer F.Cu) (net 30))
 (via (at 92.329 105.664) (size 1.4) (drill 0.6) (layers F.Cu B.Cu) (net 20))
 (segment (start 86.64 105.664) (end 92.329 105.664) (width 2) (layer F.Cu) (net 20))
 (segment (start 95.758 105.664) (end 95.758 102.616) (width 1.4) (layer F.Cu) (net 20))
 (segment (start 95.758 105.664) (end 92.329 105.664) (width 1.4) (layer F.Cu) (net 20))
 (segment (start 95.123 102.616) (end 95.758 102.616) (width 1.4) (layer F.Cu) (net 20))
 (segment (start 95.106 102.599) (end 95.123 102.616) (width 0.3) (layer F.Cu) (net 20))
 (segment (start 94.742 102.599) (end 95.106 102.599) (width 0.3) (layer F.Cu) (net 20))
 (segment (start 92.329 105.664) (end 94.107 105.664) (width 1.4) (layer B.Cu) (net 20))
 (via (at 97.663 105.664) (size 1.4) (drill 0.6) (layers F.Cu B.Cu) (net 25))
 (segment (start 97.663 105.664) (end 100.07579 105.664) (width 1.4) (layer F.Cu) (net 25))
 (segment (start 97.663 105.664) (end 95.932 105.664) (width 1.4) (layer B.Cu) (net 25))
 (segment (start 99.888 105.476) (end 100.076 105.664) (width 1.4) (layer F.Cu) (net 25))
 (segment (start 99.888 101.076) (end 99.888 105.476) (width 1.4) (layer F.Cu) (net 25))
 (via (at 88.646 103.759) (size 0.8) (drill 0.4) (layers F.Cu B.Cu) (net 24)))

